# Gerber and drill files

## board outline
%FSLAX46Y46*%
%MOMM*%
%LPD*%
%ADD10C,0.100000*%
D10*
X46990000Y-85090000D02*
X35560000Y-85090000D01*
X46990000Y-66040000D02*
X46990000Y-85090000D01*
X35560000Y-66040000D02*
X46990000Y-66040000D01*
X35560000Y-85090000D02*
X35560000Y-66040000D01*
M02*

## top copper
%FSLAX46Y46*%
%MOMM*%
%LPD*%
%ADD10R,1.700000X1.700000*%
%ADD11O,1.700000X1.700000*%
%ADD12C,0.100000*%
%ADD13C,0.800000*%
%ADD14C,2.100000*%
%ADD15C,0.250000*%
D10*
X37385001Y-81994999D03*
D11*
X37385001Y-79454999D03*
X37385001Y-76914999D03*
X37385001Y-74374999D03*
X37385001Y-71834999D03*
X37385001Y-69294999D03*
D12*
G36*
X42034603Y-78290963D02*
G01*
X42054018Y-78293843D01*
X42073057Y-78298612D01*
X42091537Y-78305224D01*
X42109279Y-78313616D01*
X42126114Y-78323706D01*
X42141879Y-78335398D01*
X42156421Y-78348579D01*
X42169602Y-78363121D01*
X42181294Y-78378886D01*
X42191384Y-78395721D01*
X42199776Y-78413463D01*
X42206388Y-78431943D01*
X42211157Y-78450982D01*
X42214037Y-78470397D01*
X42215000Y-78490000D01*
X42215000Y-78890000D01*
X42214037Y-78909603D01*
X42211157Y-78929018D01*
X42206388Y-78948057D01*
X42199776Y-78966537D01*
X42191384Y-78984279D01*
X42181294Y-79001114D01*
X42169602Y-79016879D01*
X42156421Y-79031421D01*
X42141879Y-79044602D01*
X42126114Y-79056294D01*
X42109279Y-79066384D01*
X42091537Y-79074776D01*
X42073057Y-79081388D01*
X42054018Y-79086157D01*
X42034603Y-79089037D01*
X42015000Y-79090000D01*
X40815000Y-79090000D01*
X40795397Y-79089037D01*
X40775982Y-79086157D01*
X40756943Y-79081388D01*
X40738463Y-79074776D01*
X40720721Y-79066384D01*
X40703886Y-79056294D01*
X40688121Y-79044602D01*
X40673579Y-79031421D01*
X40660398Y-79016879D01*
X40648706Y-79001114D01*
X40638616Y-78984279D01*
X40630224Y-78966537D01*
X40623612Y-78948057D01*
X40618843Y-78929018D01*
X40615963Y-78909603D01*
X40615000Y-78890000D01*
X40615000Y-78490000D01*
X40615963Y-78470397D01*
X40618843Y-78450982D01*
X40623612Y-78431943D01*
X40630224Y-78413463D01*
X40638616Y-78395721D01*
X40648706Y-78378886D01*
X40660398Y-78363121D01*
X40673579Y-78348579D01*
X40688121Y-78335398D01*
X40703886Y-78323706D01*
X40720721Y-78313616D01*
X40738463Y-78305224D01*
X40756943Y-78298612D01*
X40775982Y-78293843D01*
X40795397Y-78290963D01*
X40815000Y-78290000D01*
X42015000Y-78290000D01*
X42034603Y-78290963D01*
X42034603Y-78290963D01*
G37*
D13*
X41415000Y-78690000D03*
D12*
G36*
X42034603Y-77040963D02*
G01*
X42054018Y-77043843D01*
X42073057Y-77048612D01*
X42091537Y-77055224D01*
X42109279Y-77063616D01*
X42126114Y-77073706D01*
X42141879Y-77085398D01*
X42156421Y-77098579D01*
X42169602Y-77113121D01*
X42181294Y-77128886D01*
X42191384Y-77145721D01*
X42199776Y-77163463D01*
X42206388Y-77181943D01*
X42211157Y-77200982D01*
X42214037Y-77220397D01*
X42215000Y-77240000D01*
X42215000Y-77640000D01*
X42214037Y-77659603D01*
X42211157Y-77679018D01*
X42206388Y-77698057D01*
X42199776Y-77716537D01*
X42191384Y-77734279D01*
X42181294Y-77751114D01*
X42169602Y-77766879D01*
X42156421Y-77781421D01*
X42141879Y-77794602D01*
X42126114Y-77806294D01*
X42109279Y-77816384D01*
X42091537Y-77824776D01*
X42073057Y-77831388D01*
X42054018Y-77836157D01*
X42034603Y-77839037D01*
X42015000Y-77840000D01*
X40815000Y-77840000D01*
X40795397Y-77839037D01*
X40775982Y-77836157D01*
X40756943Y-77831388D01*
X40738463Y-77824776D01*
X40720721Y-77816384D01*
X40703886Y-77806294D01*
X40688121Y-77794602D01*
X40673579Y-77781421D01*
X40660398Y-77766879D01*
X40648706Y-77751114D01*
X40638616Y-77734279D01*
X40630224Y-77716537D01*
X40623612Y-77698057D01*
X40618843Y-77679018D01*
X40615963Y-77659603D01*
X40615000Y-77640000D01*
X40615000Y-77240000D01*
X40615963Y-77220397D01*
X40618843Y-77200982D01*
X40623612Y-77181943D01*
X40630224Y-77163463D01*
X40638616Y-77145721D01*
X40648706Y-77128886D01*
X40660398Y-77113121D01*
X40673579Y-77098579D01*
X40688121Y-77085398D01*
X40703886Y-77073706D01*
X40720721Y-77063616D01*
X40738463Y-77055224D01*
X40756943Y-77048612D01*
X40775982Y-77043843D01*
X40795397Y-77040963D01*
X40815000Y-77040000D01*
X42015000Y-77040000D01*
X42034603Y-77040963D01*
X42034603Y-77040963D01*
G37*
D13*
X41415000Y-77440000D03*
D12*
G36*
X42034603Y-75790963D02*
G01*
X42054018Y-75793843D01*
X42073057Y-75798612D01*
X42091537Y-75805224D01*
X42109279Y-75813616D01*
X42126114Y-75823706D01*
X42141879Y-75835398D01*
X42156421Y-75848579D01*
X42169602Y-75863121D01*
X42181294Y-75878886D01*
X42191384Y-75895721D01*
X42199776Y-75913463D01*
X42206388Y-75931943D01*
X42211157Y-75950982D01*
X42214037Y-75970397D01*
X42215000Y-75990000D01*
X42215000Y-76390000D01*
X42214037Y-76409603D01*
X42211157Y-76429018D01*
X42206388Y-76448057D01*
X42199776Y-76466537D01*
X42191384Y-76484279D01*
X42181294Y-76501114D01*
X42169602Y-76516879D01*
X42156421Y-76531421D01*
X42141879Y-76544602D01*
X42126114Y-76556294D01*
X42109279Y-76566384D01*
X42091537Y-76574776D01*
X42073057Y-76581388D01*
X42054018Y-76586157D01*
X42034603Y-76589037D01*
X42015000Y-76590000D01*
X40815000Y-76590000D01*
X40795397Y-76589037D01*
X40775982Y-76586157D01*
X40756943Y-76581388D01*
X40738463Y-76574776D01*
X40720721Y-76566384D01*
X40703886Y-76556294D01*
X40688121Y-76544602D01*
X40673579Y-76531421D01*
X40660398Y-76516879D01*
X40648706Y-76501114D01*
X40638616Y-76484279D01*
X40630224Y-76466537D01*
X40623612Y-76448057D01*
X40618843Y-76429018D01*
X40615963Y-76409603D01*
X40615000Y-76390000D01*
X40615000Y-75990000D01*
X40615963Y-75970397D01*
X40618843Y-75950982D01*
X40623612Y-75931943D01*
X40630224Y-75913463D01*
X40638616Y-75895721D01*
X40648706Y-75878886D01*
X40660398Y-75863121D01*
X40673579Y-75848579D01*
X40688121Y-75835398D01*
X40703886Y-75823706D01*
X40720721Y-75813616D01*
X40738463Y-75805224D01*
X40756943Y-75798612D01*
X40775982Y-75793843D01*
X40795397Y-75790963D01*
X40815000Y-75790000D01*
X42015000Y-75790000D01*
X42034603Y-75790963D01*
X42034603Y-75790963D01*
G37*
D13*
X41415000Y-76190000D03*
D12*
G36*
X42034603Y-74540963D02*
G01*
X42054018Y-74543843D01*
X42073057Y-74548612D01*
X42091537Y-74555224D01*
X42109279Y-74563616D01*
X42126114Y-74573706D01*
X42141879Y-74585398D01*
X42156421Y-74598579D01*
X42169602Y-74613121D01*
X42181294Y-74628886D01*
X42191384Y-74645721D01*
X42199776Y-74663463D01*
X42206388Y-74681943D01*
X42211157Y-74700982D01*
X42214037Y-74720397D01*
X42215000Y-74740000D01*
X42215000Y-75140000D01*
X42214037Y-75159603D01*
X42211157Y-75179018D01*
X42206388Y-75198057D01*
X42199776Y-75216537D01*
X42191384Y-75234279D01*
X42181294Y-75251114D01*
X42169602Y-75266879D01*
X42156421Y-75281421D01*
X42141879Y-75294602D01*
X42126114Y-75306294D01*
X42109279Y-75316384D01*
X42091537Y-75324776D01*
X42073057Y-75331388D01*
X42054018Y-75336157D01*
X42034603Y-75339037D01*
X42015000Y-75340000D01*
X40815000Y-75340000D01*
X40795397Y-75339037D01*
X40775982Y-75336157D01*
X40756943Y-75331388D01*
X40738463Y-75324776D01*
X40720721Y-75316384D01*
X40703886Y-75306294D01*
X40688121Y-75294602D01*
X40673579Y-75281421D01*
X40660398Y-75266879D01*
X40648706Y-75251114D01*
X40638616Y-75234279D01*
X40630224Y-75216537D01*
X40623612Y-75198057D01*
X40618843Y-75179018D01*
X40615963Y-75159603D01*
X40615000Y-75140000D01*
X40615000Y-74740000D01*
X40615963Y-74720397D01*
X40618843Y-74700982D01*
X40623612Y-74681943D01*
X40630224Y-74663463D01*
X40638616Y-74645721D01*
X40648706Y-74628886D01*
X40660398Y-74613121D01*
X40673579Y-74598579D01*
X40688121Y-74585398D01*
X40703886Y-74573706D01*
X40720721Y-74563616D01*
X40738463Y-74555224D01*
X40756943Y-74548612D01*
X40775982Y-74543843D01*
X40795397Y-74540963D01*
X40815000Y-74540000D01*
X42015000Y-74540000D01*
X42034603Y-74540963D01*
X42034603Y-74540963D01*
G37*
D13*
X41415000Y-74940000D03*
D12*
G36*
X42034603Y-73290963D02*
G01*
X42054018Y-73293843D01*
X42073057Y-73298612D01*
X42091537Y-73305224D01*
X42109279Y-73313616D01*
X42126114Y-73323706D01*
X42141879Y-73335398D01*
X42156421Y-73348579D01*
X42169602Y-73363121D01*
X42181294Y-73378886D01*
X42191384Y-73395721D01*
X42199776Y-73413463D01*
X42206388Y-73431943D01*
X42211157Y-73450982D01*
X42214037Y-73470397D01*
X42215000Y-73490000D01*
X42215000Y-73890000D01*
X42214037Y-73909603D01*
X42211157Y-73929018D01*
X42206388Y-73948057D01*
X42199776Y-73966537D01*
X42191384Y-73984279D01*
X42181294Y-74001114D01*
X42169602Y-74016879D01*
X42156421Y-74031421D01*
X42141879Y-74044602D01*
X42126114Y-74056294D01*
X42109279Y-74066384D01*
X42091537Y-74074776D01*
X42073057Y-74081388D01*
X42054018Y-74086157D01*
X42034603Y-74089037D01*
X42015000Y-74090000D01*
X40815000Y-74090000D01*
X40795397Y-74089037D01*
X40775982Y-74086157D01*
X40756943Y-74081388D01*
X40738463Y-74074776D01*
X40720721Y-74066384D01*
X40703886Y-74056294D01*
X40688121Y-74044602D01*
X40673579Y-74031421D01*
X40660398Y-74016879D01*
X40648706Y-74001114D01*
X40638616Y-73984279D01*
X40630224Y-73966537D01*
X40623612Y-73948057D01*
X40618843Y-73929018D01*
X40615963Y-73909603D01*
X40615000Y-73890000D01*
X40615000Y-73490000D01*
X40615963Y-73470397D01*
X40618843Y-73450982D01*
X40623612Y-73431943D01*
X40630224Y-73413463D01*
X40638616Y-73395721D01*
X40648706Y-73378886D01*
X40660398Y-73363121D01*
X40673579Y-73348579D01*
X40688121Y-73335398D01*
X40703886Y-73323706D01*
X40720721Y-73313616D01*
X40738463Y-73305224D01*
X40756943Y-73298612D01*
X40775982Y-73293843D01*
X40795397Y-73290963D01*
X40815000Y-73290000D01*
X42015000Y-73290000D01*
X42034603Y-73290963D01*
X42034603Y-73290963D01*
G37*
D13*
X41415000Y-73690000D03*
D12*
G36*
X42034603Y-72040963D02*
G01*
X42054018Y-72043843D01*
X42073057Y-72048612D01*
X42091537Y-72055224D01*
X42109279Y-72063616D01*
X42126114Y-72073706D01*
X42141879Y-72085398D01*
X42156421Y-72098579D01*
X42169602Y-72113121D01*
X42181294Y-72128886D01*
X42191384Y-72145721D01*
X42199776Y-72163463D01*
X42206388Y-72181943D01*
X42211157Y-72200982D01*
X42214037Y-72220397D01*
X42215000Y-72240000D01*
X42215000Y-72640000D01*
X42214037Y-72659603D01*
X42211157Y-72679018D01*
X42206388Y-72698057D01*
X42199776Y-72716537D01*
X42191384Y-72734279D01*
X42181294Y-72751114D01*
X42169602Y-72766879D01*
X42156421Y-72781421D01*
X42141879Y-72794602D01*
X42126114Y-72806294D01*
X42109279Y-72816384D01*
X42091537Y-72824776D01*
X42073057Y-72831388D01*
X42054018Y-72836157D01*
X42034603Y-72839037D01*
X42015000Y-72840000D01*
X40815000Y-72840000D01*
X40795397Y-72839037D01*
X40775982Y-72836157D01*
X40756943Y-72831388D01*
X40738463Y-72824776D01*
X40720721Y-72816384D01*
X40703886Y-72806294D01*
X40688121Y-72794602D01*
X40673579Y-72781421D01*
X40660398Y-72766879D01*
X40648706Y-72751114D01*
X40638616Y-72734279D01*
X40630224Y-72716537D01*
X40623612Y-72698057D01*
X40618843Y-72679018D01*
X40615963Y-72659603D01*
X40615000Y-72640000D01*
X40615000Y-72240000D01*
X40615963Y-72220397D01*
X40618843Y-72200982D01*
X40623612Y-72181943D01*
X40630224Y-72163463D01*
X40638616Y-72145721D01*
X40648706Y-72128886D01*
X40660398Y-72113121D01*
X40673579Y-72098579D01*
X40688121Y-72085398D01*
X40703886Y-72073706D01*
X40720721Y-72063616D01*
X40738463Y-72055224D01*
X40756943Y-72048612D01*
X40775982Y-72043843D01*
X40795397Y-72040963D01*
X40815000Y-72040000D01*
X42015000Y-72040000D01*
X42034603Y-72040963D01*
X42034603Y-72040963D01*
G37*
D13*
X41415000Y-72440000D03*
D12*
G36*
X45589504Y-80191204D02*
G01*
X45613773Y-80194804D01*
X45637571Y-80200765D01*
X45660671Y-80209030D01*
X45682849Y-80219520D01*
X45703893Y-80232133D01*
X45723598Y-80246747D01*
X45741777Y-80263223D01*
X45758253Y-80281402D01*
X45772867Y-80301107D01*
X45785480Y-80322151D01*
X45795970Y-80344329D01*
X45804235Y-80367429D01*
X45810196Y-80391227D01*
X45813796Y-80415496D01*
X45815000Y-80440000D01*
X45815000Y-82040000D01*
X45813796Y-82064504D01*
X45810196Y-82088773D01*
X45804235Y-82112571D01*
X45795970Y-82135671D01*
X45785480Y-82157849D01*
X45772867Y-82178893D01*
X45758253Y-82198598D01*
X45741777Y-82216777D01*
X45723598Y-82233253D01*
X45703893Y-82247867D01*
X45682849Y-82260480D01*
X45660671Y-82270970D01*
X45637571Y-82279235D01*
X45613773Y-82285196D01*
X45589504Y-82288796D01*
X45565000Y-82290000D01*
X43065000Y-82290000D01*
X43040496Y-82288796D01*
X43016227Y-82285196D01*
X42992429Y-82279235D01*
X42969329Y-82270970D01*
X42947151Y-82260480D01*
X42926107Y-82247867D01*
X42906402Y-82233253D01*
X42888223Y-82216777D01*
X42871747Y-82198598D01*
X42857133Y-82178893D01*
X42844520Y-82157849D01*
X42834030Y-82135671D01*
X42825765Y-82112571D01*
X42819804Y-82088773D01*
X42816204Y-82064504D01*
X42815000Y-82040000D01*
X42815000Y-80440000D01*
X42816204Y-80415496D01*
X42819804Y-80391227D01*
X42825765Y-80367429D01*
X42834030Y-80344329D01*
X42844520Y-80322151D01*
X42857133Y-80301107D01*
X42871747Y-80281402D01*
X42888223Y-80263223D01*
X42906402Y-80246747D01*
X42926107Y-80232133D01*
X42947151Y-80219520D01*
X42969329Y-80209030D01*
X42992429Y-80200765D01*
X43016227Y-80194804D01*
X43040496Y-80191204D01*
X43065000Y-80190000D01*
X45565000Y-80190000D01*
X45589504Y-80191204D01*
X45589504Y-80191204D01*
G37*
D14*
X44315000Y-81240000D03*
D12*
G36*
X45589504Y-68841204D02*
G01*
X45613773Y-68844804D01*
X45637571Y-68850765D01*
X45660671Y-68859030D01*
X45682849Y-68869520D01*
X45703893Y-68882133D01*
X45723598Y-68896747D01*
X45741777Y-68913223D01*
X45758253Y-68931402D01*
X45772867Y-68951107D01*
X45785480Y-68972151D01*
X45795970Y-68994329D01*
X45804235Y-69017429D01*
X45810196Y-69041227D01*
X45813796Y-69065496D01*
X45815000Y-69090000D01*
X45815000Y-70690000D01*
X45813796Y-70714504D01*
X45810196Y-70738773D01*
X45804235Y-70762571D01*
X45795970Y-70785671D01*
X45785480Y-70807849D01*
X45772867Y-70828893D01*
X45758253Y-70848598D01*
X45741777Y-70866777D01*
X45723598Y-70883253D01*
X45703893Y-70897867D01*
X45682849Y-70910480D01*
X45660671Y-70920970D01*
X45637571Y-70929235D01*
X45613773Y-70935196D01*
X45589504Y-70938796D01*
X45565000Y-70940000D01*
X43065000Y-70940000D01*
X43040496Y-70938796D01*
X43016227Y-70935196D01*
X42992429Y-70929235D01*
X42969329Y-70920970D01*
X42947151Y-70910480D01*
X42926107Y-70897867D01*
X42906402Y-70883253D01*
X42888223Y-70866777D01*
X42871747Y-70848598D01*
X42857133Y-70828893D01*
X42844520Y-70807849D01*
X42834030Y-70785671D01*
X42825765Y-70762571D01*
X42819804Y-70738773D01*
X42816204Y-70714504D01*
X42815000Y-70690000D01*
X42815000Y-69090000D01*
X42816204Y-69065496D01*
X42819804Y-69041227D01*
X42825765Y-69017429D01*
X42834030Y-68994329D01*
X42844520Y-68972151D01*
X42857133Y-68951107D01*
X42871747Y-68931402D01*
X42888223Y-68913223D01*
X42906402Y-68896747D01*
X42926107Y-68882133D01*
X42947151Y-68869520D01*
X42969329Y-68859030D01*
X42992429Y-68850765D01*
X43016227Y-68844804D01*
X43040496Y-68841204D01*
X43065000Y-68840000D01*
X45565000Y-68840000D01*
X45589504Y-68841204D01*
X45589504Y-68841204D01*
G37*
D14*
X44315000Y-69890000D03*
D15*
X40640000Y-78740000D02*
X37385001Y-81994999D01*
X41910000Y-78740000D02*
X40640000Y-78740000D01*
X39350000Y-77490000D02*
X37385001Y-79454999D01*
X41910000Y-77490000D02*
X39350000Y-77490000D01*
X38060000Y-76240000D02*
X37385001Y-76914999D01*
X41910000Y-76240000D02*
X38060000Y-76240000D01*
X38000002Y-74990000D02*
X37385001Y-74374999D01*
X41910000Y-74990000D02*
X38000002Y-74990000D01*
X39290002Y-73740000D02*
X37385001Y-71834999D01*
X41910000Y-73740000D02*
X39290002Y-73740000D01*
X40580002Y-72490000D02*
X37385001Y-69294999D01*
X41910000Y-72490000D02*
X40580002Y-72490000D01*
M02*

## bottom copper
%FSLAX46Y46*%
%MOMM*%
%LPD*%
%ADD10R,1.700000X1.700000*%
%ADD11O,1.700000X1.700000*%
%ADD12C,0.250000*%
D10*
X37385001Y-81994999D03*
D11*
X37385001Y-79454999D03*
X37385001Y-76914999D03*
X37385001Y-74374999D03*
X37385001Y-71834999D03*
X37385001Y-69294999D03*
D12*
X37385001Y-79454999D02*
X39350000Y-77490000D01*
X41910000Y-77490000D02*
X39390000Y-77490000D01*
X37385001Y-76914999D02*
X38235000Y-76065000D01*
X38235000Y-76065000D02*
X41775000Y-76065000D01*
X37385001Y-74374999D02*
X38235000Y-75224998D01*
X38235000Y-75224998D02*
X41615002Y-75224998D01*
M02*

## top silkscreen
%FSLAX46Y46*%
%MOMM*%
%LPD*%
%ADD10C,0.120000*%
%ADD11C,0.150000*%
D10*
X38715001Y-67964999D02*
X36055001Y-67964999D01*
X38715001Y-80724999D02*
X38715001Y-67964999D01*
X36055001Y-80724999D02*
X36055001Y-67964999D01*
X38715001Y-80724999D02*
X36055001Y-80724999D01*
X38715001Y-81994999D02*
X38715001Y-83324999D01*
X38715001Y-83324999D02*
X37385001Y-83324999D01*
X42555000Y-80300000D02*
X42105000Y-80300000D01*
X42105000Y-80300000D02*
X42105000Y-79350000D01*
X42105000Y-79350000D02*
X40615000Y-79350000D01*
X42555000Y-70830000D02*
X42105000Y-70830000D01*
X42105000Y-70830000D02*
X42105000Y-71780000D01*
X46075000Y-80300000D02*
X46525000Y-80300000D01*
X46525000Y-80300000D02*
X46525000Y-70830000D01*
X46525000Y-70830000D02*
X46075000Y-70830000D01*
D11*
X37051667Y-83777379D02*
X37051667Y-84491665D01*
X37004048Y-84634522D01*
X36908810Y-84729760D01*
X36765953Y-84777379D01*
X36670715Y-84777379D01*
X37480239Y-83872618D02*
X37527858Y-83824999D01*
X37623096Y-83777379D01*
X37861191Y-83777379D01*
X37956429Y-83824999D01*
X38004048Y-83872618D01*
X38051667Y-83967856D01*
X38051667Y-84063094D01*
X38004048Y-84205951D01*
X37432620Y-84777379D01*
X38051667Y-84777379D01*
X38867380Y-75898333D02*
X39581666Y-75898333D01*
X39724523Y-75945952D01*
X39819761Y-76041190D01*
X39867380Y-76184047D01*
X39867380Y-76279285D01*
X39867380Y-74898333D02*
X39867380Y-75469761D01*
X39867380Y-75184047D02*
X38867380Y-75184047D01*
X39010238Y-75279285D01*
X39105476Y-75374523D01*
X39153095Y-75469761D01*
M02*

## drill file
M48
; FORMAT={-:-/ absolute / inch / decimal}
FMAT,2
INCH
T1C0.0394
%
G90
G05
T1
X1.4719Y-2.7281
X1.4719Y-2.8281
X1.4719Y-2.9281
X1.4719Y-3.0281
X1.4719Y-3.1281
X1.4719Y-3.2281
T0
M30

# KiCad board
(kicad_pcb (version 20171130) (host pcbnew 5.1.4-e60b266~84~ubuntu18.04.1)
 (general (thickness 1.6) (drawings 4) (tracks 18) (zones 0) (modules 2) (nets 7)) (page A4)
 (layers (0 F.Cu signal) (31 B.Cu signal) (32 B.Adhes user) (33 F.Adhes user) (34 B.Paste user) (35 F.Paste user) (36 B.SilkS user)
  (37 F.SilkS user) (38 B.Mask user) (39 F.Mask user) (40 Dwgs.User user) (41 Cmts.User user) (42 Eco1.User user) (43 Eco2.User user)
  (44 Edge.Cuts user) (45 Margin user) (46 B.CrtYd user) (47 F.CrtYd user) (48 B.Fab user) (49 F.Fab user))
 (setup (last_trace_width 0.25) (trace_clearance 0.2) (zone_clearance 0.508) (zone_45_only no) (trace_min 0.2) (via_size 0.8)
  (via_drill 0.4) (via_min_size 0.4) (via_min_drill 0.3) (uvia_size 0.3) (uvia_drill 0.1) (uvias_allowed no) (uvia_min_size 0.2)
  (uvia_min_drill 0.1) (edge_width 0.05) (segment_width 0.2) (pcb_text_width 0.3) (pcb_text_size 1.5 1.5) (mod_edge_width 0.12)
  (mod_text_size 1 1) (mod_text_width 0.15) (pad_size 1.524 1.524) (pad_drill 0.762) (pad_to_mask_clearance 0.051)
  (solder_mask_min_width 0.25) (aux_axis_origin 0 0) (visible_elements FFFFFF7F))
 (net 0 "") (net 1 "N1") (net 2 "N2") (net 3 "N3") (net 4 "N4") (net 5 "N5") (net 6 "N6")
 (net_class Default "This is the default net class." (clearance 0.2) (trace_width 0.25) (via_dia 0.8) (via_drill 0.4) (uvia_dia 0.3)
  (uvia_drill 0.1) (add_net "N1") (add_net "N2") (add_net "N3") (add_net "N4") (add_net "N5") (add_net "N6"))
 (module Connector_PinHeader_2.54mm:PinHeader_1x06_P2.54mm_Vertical (layer F.Cu) (at 37.385001 81.994999 180)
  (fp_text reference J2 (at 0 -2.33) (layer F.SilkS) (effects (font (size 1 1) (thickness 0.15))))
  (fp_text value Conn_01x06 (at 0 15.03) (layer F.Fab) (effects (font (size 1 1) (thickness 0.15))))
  (fp_line (start -1.33 14.03) (end 1.33 14.03) (layer F.SilkS) (width 0.12))
  (fp_line (start -1.33 1.27) (end -1.33 14.03) (layer F.SilkS) (width 0.12))
  (fp_line (start 1.33 1.27) (end 1.33 14.03) (layer F.SilkS) (width 0.12))
  (fp_line (start -1.33 1.27) (end 1.33 1.27) (layer F.SilkS) (width 0.12))
  (fp_line (start -1.33 0) (end -1.33 -1.33) (layer F.SilkS) (width 0.12))
  (fp_line (start -1.33 -1.33) (end 0 -1.33) (layer F.SilkS) (width 0.12))
  (pad 1 thru_hole rect (at 0 0 180) (size 1.7 1.7) (drill 1) (layers *.Cu *.Mask) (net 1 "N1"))
  (pad 2 thru_hole oval (at 0 2.54 180) (size 1.7 1.7) (drill 1) (layers *.Cu *.Mask) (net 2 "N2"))
  (pad 3 thru_hole oval (at 0 5.08 180) (size 1.7 1.7) (drill 1) (layers *.Cu *.Mask) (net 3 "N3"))
  (pad 4 thru_hole oval (at 0 7.62 180) (size 1.7 1.7) (drill 1) (layers *.Cu *.Mask) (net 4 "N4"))
  (pad 5 thru_hole oval (at 0 10.16 180) (size 1.7 1.7) (drill 1) (layers *.Cu *.Mask) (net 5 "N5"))
  (pad 6 thru_hole oval (at 0 12.7 180) (size 1.7 1.7) (drill 1) (layers *.Cu *.Mask) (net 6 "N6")))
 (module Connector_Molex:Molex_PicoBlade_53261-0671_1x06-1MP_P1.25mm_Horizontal (layer F.Cu) (at 43.815 75.565 90)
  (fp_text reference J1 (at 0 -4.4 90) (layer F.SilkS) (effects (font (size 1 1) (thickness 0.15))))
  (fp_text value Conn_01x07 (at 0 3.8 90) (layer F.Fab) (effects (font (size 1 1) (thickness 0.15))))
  (fp_line (start -4.735 -1.26) (end -4.735 -1.71) (layer F.SilkS) (width 0.12))
  (fp_line (start -4.735 -1.71) (end -3.785 -1.71) (layer F.SilkS) (width 0.12))
  (fp_line (start -3.785 -1.71) (end -3.785 -3.2) (layer F.SilkS) (width 0.12))
  (fp_line (start 4.735 -1.26) (end 4.735 -1.71) (layer F.SilkS) (width 0.12))
  (fp_line (start 4.735 -1.71) (end 3.785 -1.71) (layer F.SilkS) (width 0.12))
  (fp_line (start -4.735 2.26) (end -4.735 2.71) (layer F.SilkS) (width 0.12))
  (fp_line (start -4.735 2.71) (end 4.735 2.71) (layer F.SilkS) (width 0.12))
  (fp_line (start 4.735 2.71) (end 4.735 2.26) (layer F.SilkS) (width 0.12))
  (pad 1 smd roundrect (at -3.125 -2.4 90) (size 0.8 1.6) (layers F.Cu F.Paste F.Mask) (roundrect_rratio 0.25) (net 1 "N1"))
  (pad 2 smd roundrect (at -1.875 -2.4 90) (size 0.8 1.6) (layers F.Cu F.Paste F.Mask) (roundrect_rratio 0.25) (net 2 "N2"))
  (pad 3 smd roundrect (at -0.625 -2.4 90) (size 0.8 1.6) (layers F.Cu F.Paste F.Mask) (roundrect_rratio 0.25) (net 3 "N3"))
  (pad 4 smd roundrect (at 0.625 -2.4 90) (size 0.8 1.6) (layers F.Cu F.Paste F.Mask) (roundrect_rratio 0.25) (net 4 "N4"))
  (pad 5 smd roundrect (at 1.875 -2.4 90) (size 0.8 1.6) (layers F.Cu F.Paste F.Mask) (roundrect_rratio 0.25) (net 5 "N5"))
  (pad 6 smd roundrect (at 3.125 -2.4 90) (size 0.8 1.6) (layers F.Cu F.Paste F.Mask) (roundrect_rratio 0.25) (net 6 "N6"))
  (pad MP smd roundrect (at -5.675 0.5 90) (size 2.1 3) (layers F.Cu F.Paste F.Mask) (roundrect_rratio 0.119048))
  (pad MP smd roundrect (at 5.675 0.5 90) (size 2.1 3) (layers F.Cu F.Paste F.Mask) (roundrect_rratio 0.119048)))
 (gr_line (start 46.99 85.09) (end 35.56 85.09) (layer Edge.Cuts) (width 0.1))
 (gr_line (start 46.99 66.04) (end 46.99 85.09) (layer Edge.Cuts) (width 0.1))
 (gr_line (start 35.56 66.04) (end 46.99 66.04) (layer Edge.Cuts) (width 0.1))
 (gr_line (start 35.56 85.09) (end 35.56 66.04) (layer Edge.Cuts) (width 0.1))
 (segment (start 40.64 78.74) (end 37.385001 81.994999) (width 0.25) (layer F.Cu) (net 1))
 (segment (start 41.91 78.74) (end 40.64 78.74) (width 0.25) (layer F.Cu) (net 1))
 (segment (start 37.385001 79.454999) (end 39.35 77.49) (width 0.25) (layer B.Cu) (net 2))
 (segment (start 41.91 77.49) (end 39.39 77.49) (width 0.25) (layer B.Cu) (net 2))
 (segment (start 39.35 77.49) (end 37.385001 79.454999) (width 0.25) (layer F.Cu) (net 2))
 (segment (start 41.91 77.49) (end 39.35 77.49) (width 0.25) (layer F.Cu) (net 2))
 (segment (start 37.385001 76.914999) (end 38.235 76.065) (width 0.25) (layer B.Cu) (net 3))
 (segment (start 38.235 76.065) (end 41.775 76.065) (width 0.25) (layer B.Cu) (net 3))
 (segment (start 38.06 76.24) (end 37.385001 76.914999) (width 0.25) (layer F.Cu) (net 3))
 (segment (start 41.91 76.24) (end 38.06 76.24) (width 0.25) (layer F.Cu) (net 3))
 (segment (start 37.385001 74.374999) (end 38.235 75.224998) (width 0.25) (layer B.Cu) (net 4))
 (segment (start 38.235 75.224998) (end 41.615002 75.224998) (width 0.25) (layer B.Cu) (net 4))
 (segment (start 38.000002 74.99) (end 37.385001 74.374999) (width 0.25) (layer F.Cu) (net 4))
 (segment (start 41.91 74.99) (end 38.000002 74.99) (width 0.25) (layer F.Cu) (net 4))
 (segment (start 39.290002 73.74) (end 37.385001 71.834999) (width 0.25) (layer F.Cu) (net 5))
 (segment (start 41.91 73.74) (end 39.290002 73.74) (width 0.25) (layer F.Cu) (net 5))
 (segment (start 40.580002 72.49) (end 37.385001 69.294999) (width 0.25) (layer F.Cu) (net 6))
 (segment (start 41.91 72.49) (end 40.580002 72.49) (width 0.25) (layer F.Cu) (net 6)))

